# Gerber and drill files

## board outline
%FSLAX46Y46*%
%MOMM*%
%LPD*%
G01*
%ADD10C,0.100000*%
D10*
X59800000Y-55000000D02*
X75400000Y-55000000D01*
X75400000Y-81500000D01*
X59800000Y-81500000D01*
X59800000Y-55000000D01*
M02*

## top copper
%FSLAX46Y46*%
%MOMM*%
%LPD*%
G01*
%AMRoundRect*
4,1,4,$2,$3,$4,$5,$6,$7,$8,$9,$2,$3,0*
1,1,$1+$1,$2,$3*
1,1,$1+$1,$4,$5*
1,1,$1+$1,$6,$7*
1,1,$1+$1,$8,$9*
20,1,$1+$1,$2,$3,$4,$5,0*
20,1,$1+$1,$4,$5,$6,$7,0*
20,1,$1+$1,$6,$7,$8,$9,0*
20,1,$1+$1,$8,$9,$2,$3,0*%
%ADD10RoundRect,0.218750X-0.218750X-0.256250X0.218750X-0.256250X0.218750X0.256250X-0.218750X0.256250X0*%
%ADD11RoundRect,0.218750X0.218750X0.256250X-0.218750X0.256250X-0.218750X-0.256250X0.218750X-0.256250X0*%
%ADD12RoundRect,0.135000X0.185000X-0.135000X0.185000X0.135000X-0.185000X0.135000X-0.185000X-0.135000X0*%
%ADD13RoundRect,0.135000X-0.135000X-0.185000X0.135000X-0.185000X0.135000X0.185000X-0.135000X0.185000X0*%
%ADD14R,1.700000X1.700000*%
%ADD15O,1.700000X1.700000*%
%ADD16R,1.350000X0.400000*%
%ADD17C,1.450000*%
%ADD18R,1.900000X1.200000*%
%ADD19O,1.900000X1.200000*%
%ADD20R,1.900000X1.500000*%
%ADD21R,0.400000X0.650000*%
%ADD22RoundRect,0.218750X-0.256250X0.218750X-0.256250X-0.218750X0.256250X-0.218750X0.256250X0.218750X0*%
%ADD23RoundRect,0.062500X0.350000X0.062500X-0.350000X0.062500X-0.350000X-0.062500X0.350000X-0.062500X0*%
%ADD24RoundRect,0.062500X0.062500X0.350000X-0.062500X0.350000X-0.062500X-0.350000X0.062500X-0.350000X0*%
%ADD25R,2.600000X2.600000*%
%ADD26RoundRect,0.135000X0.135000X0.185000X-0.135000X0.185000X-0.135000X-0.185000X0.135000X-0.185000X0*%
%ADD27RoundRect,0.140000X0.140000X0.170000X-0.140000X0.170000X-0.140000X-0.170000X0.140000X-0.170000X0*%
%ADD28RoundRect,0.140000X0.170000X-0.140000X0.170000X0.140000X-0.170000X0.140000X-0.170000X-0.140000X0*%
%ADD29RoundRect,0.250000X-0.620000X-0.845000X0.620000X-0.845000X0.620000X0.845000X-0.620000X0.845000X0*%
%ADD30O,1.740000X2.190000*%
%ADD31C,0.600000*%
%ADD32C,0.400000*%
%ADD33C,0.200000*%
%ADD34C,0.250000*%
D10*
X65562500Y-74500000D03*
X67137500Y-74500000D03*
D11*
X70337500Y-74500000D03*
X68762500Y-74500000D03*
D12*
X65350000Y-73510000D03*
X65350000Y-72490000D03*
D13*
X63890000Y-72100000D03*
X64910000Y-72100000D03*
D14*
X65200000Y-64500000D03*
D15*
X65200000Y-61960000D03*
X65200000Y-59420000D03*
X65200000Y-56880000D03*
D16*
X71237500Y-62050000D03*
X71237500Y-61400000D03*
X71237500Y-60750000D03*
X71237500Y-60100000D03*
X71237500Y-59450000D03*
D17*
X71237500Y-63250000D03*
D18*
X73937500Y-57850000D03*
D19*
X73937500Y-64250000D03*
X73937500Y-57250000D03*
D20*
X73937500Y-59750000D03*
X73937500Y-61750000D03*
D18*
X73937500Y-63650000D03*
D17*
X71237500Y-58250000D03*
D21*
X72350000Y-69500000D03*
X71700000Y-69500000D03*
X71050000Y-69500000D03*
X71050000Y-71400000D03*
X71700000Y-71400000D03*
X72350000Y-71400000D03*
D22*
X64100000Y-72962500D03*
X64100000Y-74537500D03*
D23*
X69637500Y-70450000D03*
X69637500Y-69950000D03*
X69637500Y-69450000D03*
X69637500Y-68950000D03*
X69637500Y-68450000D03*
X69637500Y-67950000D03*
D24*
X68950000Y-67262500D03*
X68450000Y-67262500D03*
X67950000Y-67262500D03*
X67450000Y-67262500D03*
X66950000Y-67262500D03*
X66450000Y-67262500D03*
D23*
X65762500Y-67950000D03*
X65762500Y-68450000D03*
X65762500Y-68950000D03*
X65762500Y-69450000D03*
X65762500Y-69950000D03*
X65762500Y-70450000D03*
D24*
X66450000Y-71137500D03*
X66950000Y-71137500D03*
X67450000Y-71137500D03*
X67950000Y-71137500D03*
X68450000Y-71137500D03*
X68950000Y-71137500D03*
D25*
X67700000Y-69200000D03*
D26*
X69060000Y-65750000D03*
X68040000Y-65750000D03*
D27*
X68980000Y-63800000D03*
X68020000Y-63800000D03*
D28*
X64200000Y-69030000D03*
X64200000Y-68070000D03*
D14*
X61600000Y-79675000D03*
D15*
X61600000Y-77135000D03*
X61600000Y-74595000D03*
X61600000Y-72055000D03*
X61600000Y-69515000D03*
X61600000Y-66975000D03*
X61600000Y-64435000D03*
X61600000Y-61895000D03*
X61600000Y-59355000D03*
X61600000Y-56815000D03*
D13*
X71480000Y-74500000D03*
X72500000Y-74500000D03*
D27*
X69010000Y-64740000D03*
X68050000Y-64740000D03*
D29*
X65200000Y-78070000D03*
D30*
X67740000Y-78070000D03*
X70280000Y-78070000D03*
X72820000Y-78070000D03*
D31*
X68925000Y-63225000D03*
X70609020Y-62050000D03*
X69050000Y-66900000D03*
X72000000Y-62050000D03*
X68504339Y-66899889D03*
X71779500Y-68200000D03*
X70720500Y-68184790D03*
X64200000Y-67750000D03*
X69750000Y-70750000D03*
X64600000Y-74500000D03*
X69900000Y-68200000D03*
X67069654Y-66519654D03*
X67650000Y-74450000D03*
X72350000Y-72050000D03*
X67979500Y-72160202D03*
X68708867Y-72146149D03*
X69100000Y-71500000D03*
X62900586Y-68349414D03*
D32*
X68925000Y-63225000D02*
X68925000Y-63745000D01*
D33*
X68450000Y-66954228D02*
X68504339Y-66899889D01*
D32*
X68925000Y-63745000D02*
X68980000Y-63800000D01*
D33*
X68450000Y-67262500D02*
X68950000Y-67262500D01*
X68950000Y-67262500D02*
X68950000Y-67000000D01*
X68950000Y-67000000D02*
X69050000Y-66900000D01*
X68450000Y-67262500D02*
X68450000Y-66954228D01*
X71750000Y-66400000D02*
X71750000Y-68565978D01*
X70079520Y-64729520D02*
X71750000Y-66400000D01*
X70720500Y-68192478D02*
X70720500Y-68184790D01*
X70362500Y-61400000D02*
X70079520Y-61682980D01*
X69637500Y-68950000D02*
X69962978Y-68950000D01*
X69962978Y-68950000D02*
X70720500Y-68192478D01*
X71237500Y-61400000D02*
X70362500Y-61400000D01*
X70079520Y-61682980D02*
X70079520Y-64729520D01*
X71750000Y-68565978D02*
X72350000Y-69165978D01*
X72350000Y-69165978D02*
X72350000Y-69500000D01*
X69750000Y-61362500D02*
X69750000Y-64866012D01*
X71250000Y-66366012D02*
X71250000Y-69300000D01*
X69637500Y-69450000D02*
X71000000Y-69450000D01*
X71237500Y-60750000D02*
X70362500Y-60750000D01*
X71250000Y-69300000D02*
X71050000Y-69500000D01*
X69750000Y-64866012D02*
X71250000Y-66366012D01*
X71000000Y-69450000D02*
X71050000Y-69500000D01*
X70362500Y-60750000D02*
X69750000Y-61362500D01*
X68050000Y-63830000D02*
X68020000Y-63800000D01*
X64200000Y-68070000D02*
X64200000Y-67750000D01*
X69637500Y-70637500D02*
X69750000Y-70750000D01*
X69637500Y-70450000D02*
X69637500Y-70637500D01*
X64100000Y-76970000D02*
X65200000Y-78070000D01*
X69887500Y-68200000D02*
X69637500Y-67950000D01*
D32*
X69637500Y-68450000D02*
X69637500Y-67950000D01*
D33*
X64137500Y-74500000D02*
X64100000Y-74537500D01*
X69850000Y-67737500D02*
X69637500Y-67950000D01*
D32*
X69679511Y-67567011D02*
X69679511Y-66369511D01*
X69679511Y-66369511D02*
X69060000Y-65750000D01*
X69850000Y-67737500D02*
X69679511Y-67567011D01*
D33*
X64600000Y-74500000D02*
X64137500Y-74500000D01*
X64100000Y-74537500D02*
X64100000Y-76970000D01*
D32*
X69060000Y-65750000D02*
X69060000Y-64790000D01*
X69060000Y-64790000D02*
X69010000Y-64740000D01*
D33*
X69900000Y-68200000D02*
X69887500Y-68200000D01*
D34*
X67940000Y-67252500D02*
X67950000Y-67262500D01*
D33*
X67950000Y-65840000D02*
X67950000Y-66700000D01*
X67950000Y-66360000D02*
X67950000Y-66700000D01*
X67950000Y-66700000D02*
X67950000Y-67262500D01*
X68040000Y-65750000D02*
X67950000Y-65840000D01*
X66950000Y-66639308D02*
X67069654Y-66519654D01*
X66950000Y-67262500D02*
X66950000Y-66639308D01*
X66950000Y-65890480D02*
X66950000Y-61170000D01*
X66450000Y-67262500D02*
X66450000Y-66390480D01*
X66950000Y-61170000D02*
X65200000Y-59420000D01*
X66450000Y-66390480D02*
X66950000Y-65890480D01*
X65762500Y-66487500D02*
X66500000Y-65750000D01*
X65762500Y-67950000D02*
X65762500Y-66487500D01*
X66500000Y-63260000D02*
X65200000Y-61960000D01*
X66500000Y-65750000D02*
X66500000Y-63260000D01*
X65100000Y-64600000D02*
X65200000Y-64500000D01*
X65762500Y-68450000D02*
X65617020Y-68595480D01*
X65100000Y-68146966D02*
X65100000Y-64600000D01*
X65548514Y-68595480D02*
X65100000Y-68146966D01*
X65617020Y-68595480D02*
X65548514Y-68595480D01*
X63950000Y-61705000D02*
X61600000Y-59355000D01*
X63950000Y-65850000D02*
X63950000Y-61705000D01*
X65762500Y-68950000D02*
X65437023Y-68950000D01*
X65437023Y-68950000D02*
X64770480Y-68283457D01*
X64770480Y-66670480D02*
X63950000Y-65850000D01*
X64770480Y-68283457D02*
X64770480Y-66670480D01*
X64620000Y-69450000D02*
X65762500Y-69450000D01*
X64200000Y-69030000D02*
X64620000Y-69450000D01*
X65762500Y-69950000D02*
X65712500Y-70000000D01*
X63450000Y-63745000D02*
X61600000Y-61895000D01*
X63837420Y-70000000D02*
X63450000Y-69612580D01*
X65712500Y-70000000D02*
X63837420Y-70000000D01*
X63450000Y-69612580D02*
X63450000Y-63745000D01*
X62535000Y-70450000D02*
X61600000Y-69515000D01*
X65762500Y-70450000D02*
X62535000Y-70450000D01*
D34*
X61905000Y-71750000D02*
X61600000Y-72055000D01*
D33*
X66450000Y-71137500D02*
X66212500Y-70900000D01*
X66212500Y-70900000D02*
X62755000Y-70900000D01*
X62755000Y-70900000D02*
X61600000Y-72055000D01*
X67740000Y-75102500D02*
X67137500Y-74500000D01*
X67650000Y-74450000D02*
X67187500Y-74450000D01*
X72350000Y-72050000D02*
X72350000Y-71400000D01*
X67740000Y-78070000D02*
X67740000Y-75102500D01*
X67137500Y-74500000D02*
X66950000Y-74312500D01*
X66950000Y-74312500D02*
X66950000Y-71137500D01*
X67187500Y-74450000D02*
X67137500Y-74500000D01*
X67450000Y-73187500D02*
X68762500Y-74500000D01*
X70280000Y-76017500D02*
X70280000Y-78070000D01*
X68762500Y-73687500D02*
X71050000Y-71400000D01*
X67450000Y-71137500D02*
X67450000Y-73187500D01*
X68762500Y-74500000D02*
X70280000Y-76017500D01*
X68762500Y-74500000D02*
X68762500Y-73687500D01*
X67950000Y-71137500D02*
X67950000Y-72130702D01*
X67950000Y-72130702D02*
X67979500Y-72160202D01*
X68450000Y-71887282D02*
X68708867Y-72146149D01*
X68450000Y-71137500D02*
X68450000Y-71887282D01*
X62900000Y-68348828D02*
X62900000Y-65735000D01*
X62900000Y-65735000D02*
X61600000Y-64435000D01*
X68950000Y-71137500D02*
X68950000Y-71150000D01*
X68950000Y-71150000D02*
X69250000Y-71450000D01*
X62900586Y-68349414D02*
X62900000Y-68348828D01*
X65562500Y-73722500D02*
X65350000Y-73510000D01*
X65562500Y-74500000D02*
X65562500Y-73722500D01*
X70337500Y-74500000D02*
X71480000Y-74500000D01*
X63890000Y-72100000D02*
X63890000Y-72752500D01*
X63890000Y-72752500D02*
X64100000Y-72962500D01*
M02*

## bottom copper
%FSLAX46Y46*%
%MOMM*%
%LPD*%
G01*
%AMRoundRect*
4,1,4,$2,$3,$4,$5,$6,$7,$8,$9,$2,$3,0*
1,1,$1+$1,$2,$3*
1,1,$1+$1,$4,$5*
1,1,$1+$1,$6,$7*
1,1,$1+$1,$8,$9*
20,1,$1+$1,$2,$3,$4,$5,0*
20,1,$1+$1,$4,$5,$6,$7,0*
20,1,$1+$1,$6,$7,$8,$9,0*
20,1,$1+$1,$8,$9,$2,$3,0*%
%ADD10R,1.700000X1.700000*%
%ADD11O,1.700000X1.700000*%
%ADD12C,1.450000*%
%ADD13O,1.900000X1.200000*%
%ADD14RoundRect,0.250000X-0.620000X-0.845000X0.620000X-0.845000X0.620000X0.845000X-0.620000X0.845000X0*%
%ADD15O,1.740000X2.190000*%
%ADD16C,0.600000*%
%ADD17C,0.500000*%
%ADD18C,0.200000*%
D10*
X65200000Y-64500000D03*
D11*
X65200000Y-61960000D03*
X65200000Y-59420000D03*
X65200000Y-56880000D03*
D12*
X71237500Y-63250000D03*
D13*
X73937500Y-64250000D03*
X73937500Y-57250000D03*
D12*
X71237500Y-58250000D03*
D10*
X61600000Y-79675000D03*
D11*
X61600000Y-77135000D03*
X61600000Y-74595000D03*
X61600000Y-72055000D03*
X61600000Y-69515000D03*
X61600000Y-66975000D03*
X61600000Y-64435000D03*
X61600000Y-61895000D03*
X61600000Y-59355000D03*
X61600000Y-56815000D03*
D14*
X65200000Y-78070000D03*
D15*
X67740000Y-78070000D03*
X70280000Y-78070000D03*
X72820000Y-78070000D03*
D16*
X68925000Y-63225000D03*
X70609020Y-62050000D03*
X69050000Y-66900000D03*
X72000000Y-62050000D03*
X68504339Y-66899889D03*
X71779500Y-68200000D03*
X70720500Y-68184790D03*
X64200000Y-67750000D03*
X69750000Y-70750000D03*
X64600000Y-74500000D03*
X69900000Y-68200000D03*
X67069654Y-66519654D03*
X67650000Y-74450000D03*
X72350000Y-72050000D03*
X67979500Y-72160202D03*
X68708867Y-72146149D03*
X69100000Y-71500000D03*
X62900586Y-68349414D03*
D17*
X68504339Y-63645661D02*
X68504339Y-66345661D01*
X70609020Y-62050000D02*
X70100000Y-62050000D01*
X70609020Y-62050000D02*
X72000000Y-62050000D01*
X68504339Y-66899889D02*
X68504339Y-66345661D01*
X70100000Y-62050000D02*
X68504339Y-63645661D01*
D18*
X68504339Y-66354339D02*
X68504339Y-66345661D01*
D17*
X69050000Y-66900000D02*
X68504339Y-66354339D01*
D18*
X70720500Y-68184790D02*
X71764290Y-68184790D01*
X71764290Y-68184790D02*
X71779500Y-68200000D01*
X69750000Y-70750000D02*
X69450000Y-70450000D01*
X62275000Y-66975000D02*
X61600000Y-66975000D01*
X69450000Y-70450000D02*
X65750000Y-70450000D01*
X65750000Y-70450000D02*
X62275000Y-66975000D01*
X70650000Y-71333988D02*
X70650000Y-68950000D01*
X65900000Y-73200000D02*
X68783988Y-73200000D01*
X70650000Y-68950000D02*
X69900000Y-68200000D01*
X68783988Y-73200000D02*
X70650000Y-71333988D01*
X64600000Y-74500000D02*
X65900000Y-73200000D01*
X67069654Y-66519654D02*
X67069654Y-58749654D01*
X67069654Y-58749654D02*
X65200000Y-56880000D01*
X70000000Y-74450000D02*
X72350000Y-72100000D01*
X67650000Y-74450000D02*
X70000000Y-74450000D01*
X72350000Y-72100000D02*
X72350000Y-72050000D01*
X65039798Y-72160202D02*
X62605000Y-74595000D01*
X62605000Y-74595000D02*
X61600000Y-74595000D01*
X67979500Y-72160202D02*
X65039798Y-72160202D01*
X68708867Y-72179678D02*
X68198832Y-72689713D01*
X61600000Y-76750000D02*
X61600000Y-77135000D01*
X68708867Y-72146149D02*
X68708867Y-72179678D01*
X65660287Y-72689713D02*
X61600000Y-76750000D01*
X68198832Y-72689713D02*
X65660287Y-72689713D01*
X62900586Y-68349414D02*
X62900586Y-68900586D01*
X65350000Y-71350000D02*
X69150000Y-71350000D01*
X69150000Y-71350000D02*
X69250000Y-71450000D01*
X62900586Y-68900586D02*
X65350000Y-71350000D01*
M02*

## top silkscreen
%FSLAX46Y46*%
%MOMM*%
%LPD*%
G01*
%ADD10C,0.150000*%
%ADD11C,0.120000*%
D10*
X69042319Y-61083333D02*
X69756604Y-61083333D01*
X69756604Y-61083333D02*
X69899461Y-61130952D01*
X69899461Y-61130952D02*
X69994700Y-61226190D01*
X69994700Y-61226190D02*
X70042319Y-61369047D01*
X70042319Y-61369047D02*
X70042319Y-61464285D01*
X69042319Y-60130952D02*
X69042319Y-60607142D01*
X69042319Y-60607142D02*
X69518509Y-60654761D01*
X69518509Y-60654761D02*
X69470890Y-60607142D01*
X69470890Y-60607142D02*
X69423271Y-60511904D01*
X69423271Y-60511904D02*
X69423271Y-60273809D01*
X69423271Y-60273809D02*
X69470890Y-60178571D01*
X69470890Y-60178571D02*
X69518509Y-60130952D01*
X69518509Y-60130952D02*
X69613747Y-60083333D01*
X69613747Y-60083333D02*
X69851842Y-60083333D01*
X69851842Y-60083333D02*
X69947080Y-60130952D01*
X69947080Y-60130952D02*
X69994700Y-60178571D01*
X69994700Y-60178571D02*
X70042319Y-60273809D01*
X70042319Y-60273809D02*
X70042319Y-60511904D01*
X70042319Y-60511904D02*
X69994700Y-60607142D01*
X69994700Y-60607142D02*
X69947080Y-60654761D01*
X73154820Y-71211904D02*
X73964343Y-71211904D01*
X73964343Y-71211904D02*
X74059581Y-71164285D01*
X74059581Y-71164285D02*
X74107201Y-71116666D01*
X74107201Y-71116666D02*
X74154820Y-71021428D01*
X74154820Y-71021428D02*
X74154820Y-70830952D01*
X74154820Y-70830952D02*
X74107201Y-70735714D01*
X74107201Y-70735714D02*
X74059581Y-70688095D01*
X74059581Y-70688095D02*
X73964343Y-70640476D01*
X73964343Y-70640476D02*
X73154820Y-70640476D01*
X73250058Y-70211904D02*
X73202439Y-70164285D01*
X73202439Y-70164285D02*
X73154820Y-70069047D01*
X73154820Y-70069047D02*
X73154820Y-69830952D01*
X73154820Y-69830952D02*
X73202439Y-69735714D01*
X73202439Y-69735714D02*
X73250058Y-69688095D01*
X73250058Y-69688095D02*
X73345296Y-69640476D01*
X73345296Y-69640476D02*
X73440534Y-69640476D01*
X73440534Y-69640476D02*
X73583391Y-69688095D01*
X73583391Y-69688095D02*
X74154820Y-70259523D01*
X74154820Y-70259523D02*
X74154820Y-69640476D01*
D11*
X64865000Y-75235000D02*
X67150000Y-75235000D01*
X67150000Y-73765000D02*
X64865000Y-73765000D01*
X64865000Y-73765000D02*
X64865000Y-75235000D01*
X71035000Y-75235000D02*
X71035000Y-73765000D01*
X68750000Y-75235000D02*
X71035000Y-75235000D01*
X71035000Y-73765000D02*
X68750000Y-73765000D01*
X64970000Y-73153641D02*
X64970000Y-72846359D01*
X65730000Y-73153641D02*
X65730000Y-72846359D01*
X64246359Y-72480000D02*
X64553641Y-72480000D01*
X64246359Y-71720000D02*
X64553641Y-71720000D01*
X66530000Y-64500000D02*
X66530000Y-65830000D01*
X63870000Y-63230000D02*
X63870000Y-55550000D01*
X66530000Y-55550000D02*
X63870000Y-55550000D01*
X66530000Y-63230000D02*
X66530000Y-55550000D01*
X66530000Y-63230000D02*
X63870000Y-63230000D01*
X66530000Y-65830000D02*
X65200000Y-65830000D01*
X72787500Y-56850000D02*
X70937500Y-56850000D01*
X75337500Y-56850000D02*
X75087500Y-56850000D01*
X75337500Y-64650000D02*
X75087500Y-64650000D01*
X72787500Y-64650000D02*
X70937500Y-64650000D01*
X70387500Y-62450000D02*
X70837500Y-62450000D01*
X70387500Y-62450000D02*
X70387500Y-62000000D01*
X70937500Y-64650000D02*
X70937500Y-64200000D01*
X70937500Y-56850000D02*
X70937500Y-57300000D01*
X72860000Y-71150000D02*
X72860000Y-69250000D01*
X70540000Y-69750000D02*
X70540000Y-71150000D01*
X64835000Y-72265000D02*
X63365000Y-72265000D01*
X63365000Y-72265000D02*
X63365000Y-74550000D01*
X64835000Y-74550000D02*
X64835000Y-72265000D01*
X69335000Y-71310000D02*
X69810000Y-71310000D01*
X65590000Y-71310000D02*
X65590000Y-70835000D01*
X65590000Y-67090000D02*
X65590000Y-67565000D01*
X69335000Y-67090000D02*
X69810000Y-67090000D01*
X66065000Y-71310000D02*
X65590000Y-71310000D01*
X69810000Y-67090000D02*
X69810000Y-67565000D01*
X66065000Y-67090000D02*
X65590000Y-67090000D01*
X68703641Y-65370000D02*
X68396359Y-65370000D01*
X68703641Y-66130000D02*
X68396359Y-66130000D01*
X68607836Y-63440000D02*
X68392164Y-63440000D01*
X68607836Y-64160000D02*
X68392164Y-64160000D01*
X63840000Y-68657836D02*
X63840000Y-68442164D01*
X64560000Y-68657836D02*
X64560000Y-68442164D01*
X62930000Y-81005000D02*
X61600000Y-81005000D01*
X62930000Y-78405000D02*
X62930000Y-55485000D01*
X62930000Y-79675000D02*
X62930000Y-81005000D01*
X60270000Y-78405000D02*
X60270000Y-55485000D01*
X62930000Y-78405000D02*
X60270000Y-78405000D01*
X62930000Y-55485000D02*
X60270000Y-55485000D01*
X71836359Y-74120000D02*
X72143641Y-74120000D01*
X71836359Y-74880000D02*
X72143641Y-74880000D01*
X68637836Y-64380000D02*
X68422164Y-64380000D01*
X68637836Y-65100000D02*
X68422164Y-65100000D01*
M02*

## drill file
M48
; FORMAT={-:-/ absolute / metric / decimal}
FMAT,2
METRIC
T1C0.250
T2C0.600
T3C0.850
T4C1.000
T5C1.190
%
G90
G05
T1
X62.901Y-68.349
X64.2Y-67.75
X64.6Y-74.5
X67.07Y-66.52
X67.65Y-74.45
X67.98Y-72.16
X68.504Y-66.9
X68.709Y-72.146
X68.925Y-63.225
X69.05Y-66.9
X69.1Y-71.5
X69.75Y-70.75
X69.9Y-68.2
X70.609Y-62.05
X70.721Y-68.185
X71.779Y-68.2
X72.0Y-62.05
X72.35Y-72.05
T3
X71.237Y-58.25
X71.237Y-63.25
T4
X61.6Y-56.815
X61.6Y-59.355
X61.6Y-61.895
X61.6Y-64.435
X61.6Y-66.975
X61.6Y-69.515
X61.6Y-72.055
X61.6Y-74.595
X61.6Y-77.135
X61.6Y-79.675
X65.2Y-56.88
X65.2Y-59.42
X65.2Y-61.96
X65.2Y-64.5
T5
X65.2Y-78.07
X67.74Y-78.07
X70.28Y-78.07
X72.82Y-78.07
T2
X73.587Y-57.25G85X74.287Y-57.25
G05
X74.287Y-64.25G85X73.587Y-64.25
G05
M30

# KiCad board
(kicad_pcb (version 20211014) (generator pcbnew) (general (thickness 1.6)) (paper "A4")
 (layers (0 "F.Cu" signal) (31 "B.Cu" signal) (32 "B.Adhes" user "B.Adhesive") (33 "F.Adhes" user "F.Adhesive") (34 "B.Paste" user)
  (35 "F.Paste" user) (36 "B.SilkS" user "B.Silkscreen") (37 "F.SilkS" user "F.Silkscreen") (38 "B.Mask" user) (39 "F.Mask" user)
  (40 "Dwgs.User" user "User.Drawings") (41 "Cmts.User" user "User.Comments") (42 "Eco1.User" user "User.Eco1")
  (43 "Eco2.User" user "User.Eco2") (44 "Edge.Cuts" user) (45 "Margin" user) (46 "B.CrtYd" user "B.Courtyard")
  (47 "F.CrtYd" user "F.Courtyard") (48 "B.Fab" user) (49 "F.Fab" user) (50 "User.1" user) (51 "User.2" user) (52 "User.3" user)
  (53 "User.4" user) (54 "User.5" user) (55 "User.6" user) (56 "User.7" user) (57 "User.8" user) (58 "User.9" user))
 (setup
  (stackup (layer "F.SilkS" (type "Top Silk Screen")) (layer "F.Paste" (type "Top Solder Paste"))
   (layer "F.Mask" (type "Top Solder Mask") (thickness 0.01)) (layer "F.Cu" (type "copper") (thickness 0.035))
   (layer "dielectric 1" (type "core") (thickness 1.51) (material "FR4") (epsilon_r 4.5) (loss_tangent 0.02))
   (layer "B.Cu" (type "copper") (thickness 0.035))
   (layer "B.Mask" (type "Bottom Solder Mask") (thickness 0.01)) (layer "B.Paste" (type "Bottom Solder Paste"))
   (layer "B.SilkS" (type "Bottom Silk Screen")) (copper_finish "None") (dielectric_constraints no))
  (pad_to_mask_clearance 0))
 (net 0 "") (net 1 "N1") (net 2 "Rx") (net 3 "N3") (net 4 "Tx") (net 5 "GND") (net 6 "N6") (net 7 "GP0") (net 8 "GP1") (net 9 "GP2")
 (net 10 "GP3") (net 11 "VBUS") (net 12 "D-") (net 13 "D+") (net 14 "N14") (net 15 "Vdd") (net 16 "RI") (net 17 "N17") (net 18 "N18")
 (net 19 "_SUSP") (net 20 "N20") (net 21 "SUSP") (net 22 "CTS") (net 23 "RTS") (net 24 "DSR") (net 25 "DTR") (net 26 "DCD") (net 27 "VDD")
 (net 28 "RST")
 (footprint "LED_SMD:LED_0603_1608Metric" (layer "F.Cu") (at 66.35 74.5)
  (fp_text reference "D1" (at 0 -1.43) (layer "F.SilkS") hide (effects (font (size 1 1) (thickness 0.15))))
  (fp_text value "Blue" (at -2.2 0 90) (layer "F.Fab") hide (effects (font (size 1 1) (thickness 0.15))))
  (fp_line (start -1.485 0.735) (end 0.8 0.735) (layer "F.SilkS") (width 0.12))
  (fp_line (start 0.8 -0.735) (end -1.485 -0.735) (layer "F.SilkS") (width 0.12))
  (fp_line (start -1.485 -0.735) (end -1.485 0.735) (layer "F.SilkS") (width 0.12))
  (pad "1" smd roundrect locked (at -0.7875 0) (size 0.875 0.95) (layers "F.Cu" "F.Paste" "F.Mask") (roundrect_rratio 0.25) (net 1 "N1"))
  (pad "2" smd roundrect locked (at 0.7875 0) (size 0.875 0.95) (layers "F.Cu" "F.Paste" "F.Mask") (roundrect_rratio 0.25) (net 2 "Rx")))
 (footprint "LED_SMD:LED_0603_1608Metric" (layer "F.Cu") (at 69.55 74.5 180)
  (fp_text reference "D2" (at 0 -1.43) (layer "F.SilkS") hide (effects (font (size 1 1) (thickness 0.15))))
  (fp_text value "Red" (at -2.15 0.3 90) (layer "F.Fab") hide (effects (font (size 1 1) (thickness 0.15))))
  (fp_line (start -1.485 -0.735) (end -1.485 0.735) (layer "F.SilkS") (width 0.12))
  (fp_line (start 0.8 -0.735) (end -1.485 -0.735) (layer "F.SilkS") (width 0.12))
  (fp_line (start -1.485 0.735) (end 0.8 0.735) (layer "F.SilkS") (width 0.12))
  (pad "1" smd roundrect locked (at -0.7875 0 180) (size 0.875 0.95) (layers "F.Cu" "F.Paste" "F.Mask") (roundrect_rratio 0.25) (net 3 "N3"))
  (pad "2" smd roundrect locked (at 0.7875 0 180) (size 0.875 0.95) (layers "F.Cu" "F.Paste" "F.Mask") (roundrect_rratio 0.25) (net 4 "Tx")))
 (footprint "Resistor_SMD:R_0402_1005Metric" (layer "F.Cu") (at 65.35 73 90)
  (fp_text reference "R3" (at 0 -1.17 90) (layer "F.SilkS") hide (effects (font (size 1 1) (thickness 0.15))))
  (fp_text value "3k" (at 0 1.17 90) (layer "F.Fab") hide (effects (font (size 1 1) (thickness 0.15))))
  (fp_line (start -0.153641 -0.38) (end 0.153641 -0.38) (layer "F.SilkS") (width 0.12))
  (fp_line (start -0.153641 0.38) (end 0.153641 0.38) (layer "F.SilkS") (width 0.12))
  (pad "1" smd roundrect locked (at -0.51 0 90) (size 0.54 0.64) (layers "F.Cu" "F.Paste" "F.Mask") (roundrect_rratio 0.25) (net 1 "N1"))
  (pad "2" smd roundrect locked (at 0.51 0 90) (size 0.54 0.64) (layers "F.Cu" "F.Paste" "F.Mask") (roundrect_rratio 0.25) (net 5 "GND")))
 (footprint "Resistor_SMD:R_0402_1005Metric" (layer "F.Cu") (at 64.4 72.1)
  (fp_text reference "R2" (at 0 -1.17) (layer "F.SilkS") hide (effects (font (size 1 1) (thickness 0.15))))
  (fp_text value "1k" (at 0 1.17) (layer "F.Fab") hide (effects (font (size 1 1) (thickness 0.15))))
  (fp_line (start -0.153641 0.38) (end 0.153641 0.38) (layer "F.SilkS") (width 0.12))
  (fp_line (start -0.153641 -0.38) (end 0.153641 -0.38) (layer "F.SilkS") (width 0.12))
  (pad "1" smd roundrect locked (at -0.51 0) (size 0.54 0.64) (layers "F.Cu" "F.Paste" "F.Mask") (roundrect_rratio 0.25) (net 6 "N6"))
  (pad "2" smd roundrect locked (at 0.51 0) (size 0.54 0.64) (layers "F.Cu" "F.Paste" "F.Mask") (roundrect_rratio 0.25) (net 5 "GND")))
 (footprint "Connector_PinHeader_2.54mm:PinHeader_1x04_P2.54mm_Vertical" (layer "F.Cu") (at 65.2 64.5 180)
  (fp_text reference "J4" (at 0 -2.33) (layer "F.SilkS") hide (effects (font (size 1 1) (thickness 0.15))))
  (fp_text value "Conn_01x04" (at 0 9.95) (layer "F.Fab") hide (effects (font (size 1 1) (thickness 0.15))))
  (fp_line (start -1.33 0) (end -1.33 -1.33) (layer "F.SilkS") (width 0.12))
  (fp_line (start 1.33 1.27) (end 1.33 8.95) (layer "F.SilkS") (width 0.12))
  (fp_line (start -1.33 8.95) (end 1.33 8.95) (layer "F.SilkS") (width 0.12))
  (fp_line (start -1.33 1.27) (end -1.33 8.95) (layer "F.SilkS") (width 0.12))
  (fp_line (start -1.33 1.27) (end 1.33 1.27) (layer "F.SilkS") (width 0.12))
  (fp_line (start -1.33 -1.33) (end 0 -1.33) (layer "F.SilkS") (width 0.12))
  (pad "1" thru_hole rect locked (at 0 0 180) (size 1.7 1.7) (drill 1) (layers *.Cu *.Mask) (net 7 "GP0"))
  (pad "2" thru_hole oval locked (at 0 2.54 180) (size 1.7 1.7) (drill 1) (layers *.Cu *.Mask) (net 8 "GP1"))
  (pad "3" thru_hole oval locked (at 0 5.08 180) (size 1.7 1.7) (drill 1) (layers *.Cu *.Mask) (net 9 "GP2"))
  (pad "4" thru_hole oval locked (at 0 7.62 180) (size 1.7 1.7) (drill 1) (layers *.Cu *.Mask) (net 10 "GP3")))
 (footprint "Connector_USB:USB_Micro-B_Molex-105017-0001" (layer "F.Cu") (at 72.7 60.75 90)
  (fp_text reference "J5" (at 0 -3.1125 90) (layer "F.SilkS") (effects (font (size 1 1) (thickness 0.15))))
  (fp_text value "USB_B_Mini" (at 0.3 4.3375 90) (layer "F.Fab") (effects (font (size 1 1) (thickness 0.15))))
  (fp_line (start 3.9 0.0875) (end 3.9 -1.7625) (layer "F.SilkS") (width 0.12))
  (fp_line (start 3.9 2.6375) (end 3.9 2.3875) (layer "F.SilkS") (width 0.12))
  (fp_line (start -3.9 2.6375) (end -3.9 2.3875) (layer "F.SilkS") (width 0.12))
  (fp_line (start -3.9 0.0875) (end -3.9 -1.7625) (layer "F.SilkS") (width 0.12))
  (fp_line (start -1.7 -2.3125) (end -1.7 -1.8625) (layer "F.SilkS") (width 0.12))
  (fp_line (start -1.7 -2.3125) (end -1.25 -2.3125) (layer "F.SilkS") (width 0.12))
  (fp_line (start -3.9 -1.7625) (end -3.45 -1.7625) (layer "F.SilkS") (width 0.12))
  (fp_line (start 3.9 -1.7625) (end 3.45 -1.7625) (layer "F.SilkS") (width 0.12))
  (pad "1" smd rect locked (at -1.3 -1.4625 90) (size 0.4 1.35) (layers "F.Cu" "F.Paste" "F.Mask") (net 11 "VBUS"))
  (pad "2" smd rect locked (at -0.65 -1.4625 90) (size 0.4 1.35) (layers "F.Cu" "F.Paste" "F.Mask") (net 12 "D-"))
  (pad "3" smd rect locked (at 0 -1.4625 90) (size 0.4 1.35) (layers "F.Cu" "F.Paste" "F.Mask") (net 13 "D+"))
  (pad "4" smd rect locked (at 0.65 -1.4625 90) (size 0.4 1.35) (layers "F.Cu" "F.Paste" "F.Mask") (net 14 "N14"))
  (pad "5" smd rect locked (at 1.3 -1.4625 90) (size 0.4 1.35) (layers "F.Cu" "F.Paste" "F.Mask") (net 5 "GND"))
  (pad "6" thru_hole circle locked (at -2.5 -1.4625 90) (size 1.45 1.45) (drill 0.85) (layers *.Cu *.Mask) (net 5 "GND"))
  (pad "6" smd rect locked (at 2.9 1.2375 90) (size 1.2 1.9) (layers "F.Cu" "F.Mask") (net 5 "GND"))
  (pad "6" thru_hole oval locked (at -3.5 1.2375 270) (size 1.2 1.9) (drill oval 0.6 1.3) (layers *.Cu *.Mask) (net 5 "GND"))
  (pad "6" thru_hole oval locked (at 3.5 1.2375 90) (size 1.2 1.9) (drill oval 0.6 1.3) (layers *.Cu *.Mask) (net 5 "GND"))
  (pad "6" smd rect locked (at 1 1.2375 90) (size 1.5 1.9) (layers "F.Cu" "F.Paste" "F.Mask") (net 5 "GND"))
  (pad "6" smd rect locked (at -1 1.2375 90) (size 1.5 1.9) (layers "F.Cu" "F.Paste" "F.Mask") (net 5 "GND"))
  (pad "6" smd rect locked (at -2.9 1.2375 90) (size 1.2 1.9) (layers "F.Cu" "F.Mask") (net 5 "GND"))
  (pad "6" thru_hole circle locked (at 2.5 -1.4625 90) (size 1.45 1.45) (drill 0.85) (layers *.Cu *.Mask) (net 5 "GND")))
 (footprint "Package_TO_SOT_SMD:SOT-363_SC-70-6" (layer "F.Cu") (at 71.7 70.45 -90)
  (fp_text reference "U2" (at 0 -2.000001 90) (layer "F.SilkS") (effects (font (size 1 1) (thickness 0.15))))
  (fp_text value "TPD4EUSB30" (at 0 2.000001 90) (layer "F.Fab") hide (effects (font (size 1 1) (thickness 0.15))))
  (fp_line (start 0.7 -1.16) (end -1.2 -1.16) (layer "F.SilkS") (width 0.12))
  (fp_line (start -0.7 1.16) (end 0.7 1.16) (layer "F.SilkS") (width 0.12))
  (pad "1" smd rect locked (at -0.95 -0.65 270) (size 0.65 0.4) (layers "F.Cu" "F.Paste" "F.Mask") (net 12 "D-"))
  (pad "2" smd rect locked (at -0.95 0 270) (size 0.65 0.4) (layers "F.Cu" "F.Paste" "F.Mask") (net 5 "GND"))
  (pad "3" smd rect locked (at -0.95 0.65 270) (size 0.65 0.4) (layers "F.Cu" "F.Paste" "F.Mask") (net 13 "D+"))
  (pad "4" smd rect locked (at 0.95 0.65 270) (size 0.65 0.4) (layers "F.Cu" "F.Paste" "F.Mask") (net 4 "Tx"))
  (pad "5" smd rect locked (at 0.95 0 270) (size 0.65 0.4) (layers "F.Cu" "F.Paste" "F.Mask"))
  (pad "6" smd rect locked (at 0.95 -0.65 270) (size 0.65 0.4) (layers "F.Cu" "F.Paste" "F.Mask") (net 2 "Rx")))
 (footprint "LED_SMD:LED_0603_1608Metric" (layer "F.Cu") (at 64.1 73.75 -90)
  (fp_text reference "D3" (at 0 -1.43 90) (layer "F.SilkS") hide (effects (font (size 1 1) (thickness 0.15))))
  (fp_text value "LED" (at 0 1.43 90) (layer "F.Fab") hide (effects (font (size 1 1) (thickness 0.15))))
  (fp_line (start -1.485 -0.735) (end -1.485 0.735) (layer "F.SilkS") (width 0.12))
  (fp_line (start -1.485 0.735) (end 0.8 0.735) (layer "F.SilkS") (width 0.12))
  (fp_line (start 0.8 -0.735) (end -1.485 -0.735) (layer "F.SilkS") (width 0.12))
  (pad "1" smd roundrect locked (at -0.7875 0 270) (size 0.875 0.95) (layers "F.Cu" "F.Paste" "F.Mask") (roundrect_rratio 0.25) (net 6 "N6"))
  (pad "2" smd roundrect locked (at 0.7875 0 270) (size 0.875 0.95) (layers "F.Cu" "F.Paste" "F.Mask") (roundrect_rratio 0.25)
   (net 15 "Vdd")))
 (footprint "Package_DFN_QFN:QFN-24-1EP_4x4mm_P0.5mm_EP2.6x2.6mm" (layer "F.Cu") (at 67.7 69.2 180)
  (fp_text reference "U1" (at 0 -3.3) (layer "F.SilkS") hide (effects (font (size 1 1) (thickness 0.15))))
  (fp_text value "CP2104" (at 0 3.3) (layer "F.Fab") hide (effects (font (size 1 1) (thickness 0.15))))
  (fp_line (start -1.635 -2.11) (end -2.11 -2.11) (layer "F.SilkS") (width 0.12))
  (fp_line (start 2.11 -2.11) (end 2.11 -1.635) (layer "F.SilkS") (width 0.12))
  (fp_line (start 2.11 2.11) (end 2.11 1.635) (layer "F.SilkS") (width 0.12))
  (fp_line (start -1.635 2.11) (end -2.11 2.11) (layer "F.SilkS") (width 0.12))
  (fp_line (start 1.635 -2.11) (end 2.11 -2.11) (layer "F.SilkS") (width 0.12))
  (fp_line (start -2.11 2.11) (end -2.11 1.635) (layer "F.SilkS") (width 0.12))
  (fp_line (start 1.635 2.11) (end 2.11 2.11) (layer "F.SilkS") (width 0.12))
  (pad "" smd roundrect locked (at -0.65 -0.65 180) (size 1.05 1.05) (layers "F.Paste") (roundrect_rratio 0.238095))
  (pad "" smd roundrect locked (at 0.65 -0.65 180) (size 1.05 1.05) (layers "F.Paste") (roundrect_rratio 0.238095))
  (pad "" smd roundrect locked (at 0.65 0.65 180) (size 1.05 1.05) (layers "F.Paste") (roundrect_rratio 0.238095))
  (pad "" smd roundrect locked (at -0.65 0.65 180) (size 1.05 1.05) (layers "F.Paste") (roundrect_rratio 0.238095))
  (pad "1" smd roundrect locked (at -1.9375 -1.25 180) (size 0.825 0.25) (layers "F.Cu" "F.Paste" "F.Mask") (roundrect_rratio 0.25)
   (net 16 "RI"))
  (pad "2" smd roundrect locked (at -1.9375 -0.75 180) (size 0.825 0.25) (layers "F.Cu" "F.Paste" "F.Mask") (roundrect_rratio 0.25)
   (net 5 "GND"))
  (pad "3" smd roundrect locked (at -1.9375 -0.25 180) (size 0.825 0.25) (layers "F.Cu" "F.Paste" "F.Mask") (roundrect_rratio 0.25)
   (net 13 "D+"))
  (pad "4" smd roundrect locked (at -1.9375 0.25 180) (size 0.825 0.25) (layers "F.Cu" "F.Paste" "F.Mask") (roundrect_rratio 0.25)
   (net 12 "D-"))
  (pad "5" smd roundrect locked (at -1.9375 0.75 180) (size 0.825 0.25) (layers "F.Cu" "F.Paste" "F.Mask") (roundrect_rratio 0.25)
   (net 15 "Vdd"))
  (pad "6" smd roundrect locked (at -1.9375 1.25 180) (size 0.825 0.25) (layers "F.Cu" "F.Paste" "F.Mask") (roundrect_rratio 0.25)
   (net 15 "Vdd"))
  (pad "7" smd roundrect locked (at -1.25 1.9375 180) (size 0.25 0.825) (layers "F.Cu" "F.Paste" "F.Mask") (roundrect_rratio 0.25)
   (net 11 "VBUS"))
  (pad "8" smd roundrect locked (at -0.75 1.9375 180) (size 0.25 0.825) (layers "F.Cu" "F.Paste" "F.Mask") (roundrect_rratio 0.25)
   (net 11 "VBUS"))
  (pad "9" smd roundrect locked (at -0.25 1.9375 180) (size 0.25 0.825) (layers "F.Cu" "F.Paste" "F.Mask") (roundrect_rratio 0.25)
   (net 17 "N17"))
  (pad "10" smd roundrect locked (at 0.25 1.9375 180) (size 0.25 0.825) (layers "F.Cu" "F.Paste" "F.Mask") (roundrect_rratio 0.25)
   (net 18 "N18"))
  (pad "11" smd roundrect locked (at 0.75 1.9375 180) (size 0.25 0.825) (layers "F.Cu" "F.Paste" "F.Mask") (roundrect_rratio 0.25)
   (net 10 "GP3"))
  (pad "12" smd roundrect locked (at 1.25 1.9375 180) (size 0.25 0.825) (layers "F.Cu" "F.Paste" "F.Mask") (roundrect_rratio 0.25)
   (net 9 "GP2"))
  (pad "13" smd roundrect locked (at 1.9375 1.25 180) (size 0.825 0.25) (layers "F.Cu" "F.Paste" "F.Mask") (roundrect_rratio 0.25)
   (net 8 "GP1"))
  (pad "14" smd roundrect locked (at 1.9375 0.75 180) (size 0.825 0.25) (layers "F.Cu" "F.Paste" "F.Mask") (roundrect_rratio 0.25)
   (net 7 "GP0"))
  (pad "15" smd roundrect locked (at 1.9375 0.25 180) (size 0.825 0.25) (layers "F.Cu" "F.Paste" "F.Mask") (roundrect_rratio 0.25)
   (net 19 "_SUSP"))
  (pad "16" smd roundrect locked (at 1.9375 -0.25 180) (size 0.825 0.25) (layers "F.Cu" "F.Paste" "F.Mask") (roundrect_rratio 0.25)
   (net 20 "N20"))
  (pad "17" smd roundrect locked (at 1.9375 -0.75 180) (size 0.825 0.25) (layers "F.Cu" "F.Paste" "F.Mask") (roundrect_rratio 0.25)
   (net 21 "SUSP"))
  (pad "18" smd roundrect locked (at 1.9375 -1.25 180) (size 0.825 0.25) (layers "F.Cu" "F.Paste" "F.Mask") (roundrect_rratio 0.25)
   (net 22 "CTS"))
  (pad "19" smd roundrect locked (at 1.25 -1.9375 180) (size 0.25 0.825) (layers "F.Cu" "F.Paste" "F.Mask") (roundrect_rratio 0.25)
   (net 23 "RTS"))
  (pad "20" smd roundrect locked (at 0.75 -1.9375 180) (size 0.25 0.825) (layers "F.Cu" "F.Paste" "F.Mask") (roundrect_rratio 0.25)
   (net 2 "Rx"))
  (pad "21" smd roundrect locked (at 0.25 -1.9375 180) (size 0.25 0.825) (layers "F.Cu" "F.Paste" "F.Mask") (roundrect_rratio 0.25)
   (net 4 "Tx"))
  (pad "22" smd roundrect locked (at -0.25 -1.9375 180) (size 0.25 0.825) (layers "F.Cu" "F.Paste" "F.Mask") (roundrect_rratio 0.25)
   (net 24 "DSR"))
  (pad "23" smd roundrect locked (at -0.75 -1.9375 180) (size 0.25 0.825) (layers "F.Cu" "F.Paste" "F.Mask") (roundrect_rratio 0.25)
   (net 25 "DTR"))
  (pad "24" smd roundrect locked (at -1.25 -1.9375 180) (size 0.25 0.825) (layers "F.Cu" "F.Paste" "F.Mask") (roundrect_rratio 0.25)
   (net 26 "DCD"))
  (pad "25" smd rect locked (at 0 0 180) (size 2.6 2.6) (layers "F.Cu" "F.Mask") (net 5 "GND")))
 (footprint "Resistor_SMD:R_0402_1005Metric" (layer "F.Cu") (at 68.55 65.75 180)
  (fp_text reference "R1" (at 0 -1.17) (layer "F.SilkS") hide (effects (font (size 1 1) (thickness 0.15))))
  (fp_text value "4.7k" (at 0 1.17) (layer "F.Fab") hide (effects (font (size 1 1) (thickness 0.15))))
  (fp_line (start -0.153641 0.38) (end 0.153641 0.38) (layer "F.SilkS") (width 0.12))
  (fp_line (start -0.153641 -0.38) (end 0.153641 -0.38) (layer "F.SilkS") (width 0.12))
  (pad "1" smd roundrect locked (at -0.51 0 180) (size 0.54 0.64) (layers "F.Cu" "F.Paste" "F.Mask") (roundrect_rratio 0.25) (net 15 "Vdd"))
  (pad "2" smd roundrect locked (at 0.51 0 180) (size 0.54 0.64) (layers "F.Cu" "F.Paste" "F.Mask") (roundrect_rratio 0.25) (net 17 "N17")))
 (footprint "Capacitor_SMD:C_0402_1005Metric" (layer "F.Cu") (at 68.5 63.8 180)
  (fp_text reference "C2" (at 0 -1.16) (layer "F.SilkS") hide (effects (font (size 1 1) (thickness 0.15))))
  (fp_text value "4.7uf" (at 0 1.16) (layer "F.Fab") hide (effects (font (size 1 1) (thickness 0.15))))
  (fp_line (start -0.107836 0.36) (end 0.107836 0.36) (layer "F.SilkS") (width 0.12))
  (fp_line (start -0.107836 -0.36) (end 0.107836 -0.36) (layer "F.SilkS") (width 0.12))
  (pad "1" smd roundrect locked (at -0.48 0 180) (size 0.56 0.62) (layers "F.Cu" "F.Paste" "F.Mask") (roundrect_rratio 0.25) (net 11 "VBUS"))
  (pad "2" smd roundrect locked (at 0.48 0 180) (size 0.56 0.62) (layers "F.Cu" "F.Paste" "F.Mask") (roundrect_rratio 0.25) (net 5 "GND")))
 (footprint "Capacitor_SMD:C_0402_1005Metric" (layer "F.Cu") (at 64.2 68.55 90)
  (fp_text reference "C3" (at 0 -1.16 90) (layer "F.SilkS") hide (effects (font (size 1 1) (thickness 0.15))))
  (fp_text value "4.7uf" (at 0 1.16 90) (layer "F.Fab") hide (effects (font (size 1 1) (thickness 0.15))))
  (fp_line (start -0.107836 -0.36) (end 0.107836 -0.36) (layer "F.SilkS") (width 0.12))
  (fp_line (start -0.107836 0.36) (end 0.107836 0.36) (layer "F.SilkS") (width 0.12))
  (pad "1" smd roundrect locked (at -0.48 0 90) (size 0.56 0.62) (layers "F.Cu" "F.Paste" "F.Mask") (roundrect_rratio 0.25) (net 20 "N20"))
  (pad "2" smd roundrect locked (at 0.48 0 90) (size 0.56 0.62) (layers "F.Cu" "F.Paste" "F.Mask") (roundrect_rratio 0.25) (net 5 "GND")))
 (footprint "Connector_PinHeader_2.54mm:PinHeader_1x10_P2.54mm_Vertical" (layer "F.Cu") (at 61.6 79.675 180)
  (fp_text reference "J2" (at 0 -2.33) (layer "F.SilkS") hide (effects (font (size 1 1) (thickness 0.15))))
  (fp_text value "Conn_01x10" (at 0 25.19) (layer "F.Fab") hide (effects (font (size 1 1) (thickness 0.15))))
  (fp_line (start -1.33 -1.33) (end 0 -1.33) (layer "F.SilkS") (width 0.12))
  (fp_line (start -1.33 1.27) (end -1.33 24.19) (layer "F.SilkS") (width 0.12))
  (fp_line (start -1.33 0) (end -1.33 -1.33) (layer "F.SilkS") (width 0.12))
  (fp_line (start 1.33 1.27) (end 1.33 24.19) (layer "F.SilkS") (width 0.12))
  (fp_line (start -1.33 1.27) (end 1.33 1.27) (layer "F.SilkS") (width 0.12))
  (fp_line (start -1.33 24.19) (end 1.33 24.19) (layer "F.SilkS") (width 0.12))
  (pad "1" thru_hole rect locked (at 0 0 180) (size 1.7 1.7) (drill 1) (layers *.Cu *.Mask) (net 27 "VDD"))
  (pad "2" thru_hole oval locked (at 0 2.54 180) (size 1.7 1.7) (drill 1) (layers *.Cu *.Mask) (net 25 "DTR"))
  (pad "3" thru_hole oval locked (at 0 5.08 180) (size 1.7 1.7) (drill 1) (layers *.Cu *.Mask) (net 24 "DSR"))
  (pad "4" thru_hole oval locked (at 0 7.62 180) (size 1.7 1.7) (drill 1) (layers *.Cu *.Mask) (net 23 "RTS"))
  (pad "5" thru_hole oval locked (at 0 10.16 180) (size 1.7 1.7) (drill 1) (layers *.Cu *.Mask) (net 22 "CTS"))
  (pad "6" thru_hole oval locked (at 0 12.7 180) (size 1.7 1.7) (drill 1) (layers *.Cu *.Mask) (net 16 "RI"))
  (pad "7" thru_hole oval locked (at 0 15.24 180) (size 1.7 1.7) (drill 1) (layers *.Cu *.Mask) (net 26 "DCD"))
  (pad "8" thru_hole oval locked (at 0 17.78 180) (size 1.7 1.7) (drill 1) (layers *.Cu *.Mask) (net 21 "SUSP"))
  (pad "9" thru_hole oval locked (at 0 20.32 180) (size 1.7 1.7) (drill 1) (layers *.Cu *.Mask) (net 19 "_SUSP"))
  (pad "10" thru_hole oval locked (at 0 22.86 180) (size 1.7 1.7) (drill 1) (layers *.Cu *.Mask) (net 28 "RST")))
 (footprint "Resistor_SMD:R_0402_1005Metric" (layer "F.Cu") (at 71.99 74.5)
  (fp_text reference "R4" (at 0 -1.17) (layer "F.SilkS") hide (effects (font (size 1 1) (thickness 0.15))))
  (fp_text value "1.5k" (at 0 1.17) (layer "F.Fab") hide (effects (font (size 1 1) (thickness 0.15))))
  (fp_line (start -0.153641 -0.38) (end 0.153641 -0.38) (layer "F.SilkS") (width 0.12))
  (fp_line (start -0.153641 0.38) (end 0.153641 0.38) (layer "F.SilkS") (width 0.12))
  (pad "1" smd roundrect locked (at -0.51 0) (size 0.54 0.64) (layers "F.Cu" "F.Paste" "F.Mask") (roundrect_rratio 0.25) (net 3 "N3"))
  (pad "2" smd roundrect locked (at 0.51 0) (size 0.54 0.64) (layers "F.Cu" "F.Paste" "F.Mask") (roundrect_rratio 0.25) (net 5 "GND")))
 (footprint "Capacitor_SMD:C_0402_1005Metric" (layer "F.Cu") (at 68.53 64.74 180)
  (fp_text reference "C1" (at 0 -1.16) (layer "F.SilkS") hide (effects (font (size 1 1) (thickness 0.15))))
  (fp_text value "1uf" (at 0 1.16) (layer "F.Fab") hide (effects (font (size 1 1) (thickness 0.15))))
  (fp_line (start -0.107836 0.36) (end 0.107836 0.36) (layer "F.SilkS") (width 0.12))
  (fp_line (start -0.107836 -0.36) (end 0.107836 -0.36) (layer "F.SilkS") (width 0.12))
  (pad "1" smd roundrect locked (at -0.48 0 180) (size 0.56 0.62) (layers "F.Cu" "F.Paste" "F.Mask") (roundrect_rratio 0.25) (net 15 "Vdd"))
  (pad "2" smd roundrect locked (at 0.48 0 180) (size 0.56 0.62) (layers "F.Cu" "F.Paste" "F.Mask") (roundrect_rratio 0.25) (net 5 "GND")))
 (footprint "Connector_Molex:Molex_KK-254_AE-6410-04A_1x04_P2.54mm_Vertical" (layer "B.Cu") (at 65.2 78.07)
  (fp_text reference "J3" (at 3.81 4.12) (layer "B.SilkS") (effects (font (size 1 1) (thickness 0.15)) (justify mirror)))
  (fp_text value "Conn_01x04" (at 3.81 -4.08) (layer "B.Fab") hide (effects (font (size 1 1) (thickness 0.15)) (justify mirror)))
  (pad "1" thru_hole roundrect locked (at 0 0) (size 1.74 2.19) (drill 1.19) (layers *.Cu *.Mask) (roundrect_rratio 0.143678) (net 15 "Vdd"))
  (pad "2" thru_hole oval locked (at 2.54 0) (size 1.74 2.19) (drill 1.19) (layers *.Cu *.Mask) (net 2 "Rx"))
  (pad "3" thru_hole oval locked (at 5.08 0) (size 1.74 2.19) (drill 1.19) (layers *.Cu *.Mask) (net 4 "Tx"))
  (pad "4" thru_hole oval locked (at 7.62 0) (size 1.74 2.19) (drill 1.19) (layers *.Cu *.Mask) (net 5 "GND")))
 (gr_rect (start 59.8 55) (end 75.4 81.5) (layer "Edge.Cuts") (width 0.1) (fill none))
 (segment (start 68.925 63.225) (end 68.925 63.745) (width 0.4) (layer "F.Cu") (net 11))
 (segment (start 68.45 66.954228) (end 68.504339 66.899889) (width 0.2) (layer "F.Cu") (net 11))
 (segment (start 68.925 63.745) (end 68.98 63.8) (width 0.4) (layer "F.Cu") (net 11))
 (segment (start 68.45 67.2625) (end 68.95 67.2625) (width 0.2) (layer "F.Cu") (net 11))
 (segment (start 68.95 67.2625) (end 68.95 67) (width 0.2) (layer "F.Cu") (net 11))
 (segment (start 68.95 67) (end 69.05 66.9) (width 0.2) (layer "F.Cu") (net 11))
 (segment (start 68.45 67.2625) (end 68.45 66.954228) (width 0.2) (layer "F.Cu") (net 11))
 (via (at 68.925 63.225) (size 0.6) (drill 0.25) (layers "F.Cu" "B.Cu") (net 11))
 (via (at 70.60902 62.05) (size 0.6) (drill 0.25) (layers "F.Cu" "B.Cu") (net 11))
 (via (at 69.05 66.9) (size 0.6) (drill 0.25) (layers "F.Cu" "B.Cu") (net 11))
 (via (at 72 62.05) (size 0.6) (drill 0.25) (layers "F.Cu" "B.Cu") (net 11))
 (via (at 68.504339 66.899889) (size 0.6) (drill 0.25) (layers "F.Cu" "B.Cu") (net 11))
 (segment (start 68.504339 63.645661) (end 68.504339 66.345661) (width 0.5) (layer "B.Cu") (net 11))
 (segment (start 70.60902 62.05) (end 70.1 62.05) (width 0.5) (layer "B.Cu") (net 11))
 (segment (start 70.60902 62.05) (end 72 62.05) (width 0.5) (layer "B.Cu") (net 11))
 (segment (start 68.504339 66.899889) (end 68.504339 66.345661) (width 0.5) (layer "B.Cu") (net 11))
 (segment (start 70.1 62.05) (end 68.504339 63.645661) (width 0.5) (layer "B.Cu") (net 11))
 (segment (start 68.504339 66.354339) (end 68.504339 66.345661) (width 0.2) (layer "B.Cu") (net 11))
 (segment (start 69.05 66.9) (end 68.504339 66.354339) (width 0.5) (layer "B.Cu") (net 11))
 (segment (start 71.75 66.4) (end 71.75 68.565978) (width 0.2) (layer "F.Cu") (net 12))
 (segment (start 70.07952 64.72952) (end 71.75 66.4) (width 0.2) (layer "F.Cu") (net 12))
 (segment (start 70.7205 68.192478) (end 70.7205 68.18479) (width 0.2) (layer "F.Cu") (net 12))
 (segment (start 70.3625 61.4) (end 70.07952 61.68298) (width 0.2) (layer "F.Cu") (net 12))
 (segment (start 69.6375 68.95) (end 69.962978 68.95) (width 0.2) (layer "F.Cu") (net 12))
 (segment (start 69.962978 68.95) (end 70.7205 68.192478) (width 0.2) (layer "F.Cu") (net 12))
 (segment (start 71.2375 61.4) (end 70.3625 61.4) (width 0.2) (layer "F.Cu") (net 12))
 (segment (start 70.07952 61.68298) (end 70.07952 64.72952) (width 0.2) (layer "F.Cu") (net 12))
 (segment (start 71.75 68.565978) (end 72.35 69.165978) (width 0.2) (layer "F.Cu") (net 12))
 (segment (start 72.35 69.165978) (end 72.35 69.5) (width 0.2) (layer "F.Cu") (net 12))
 (via (at 71.7795 68.2) (size 0.6) (drill 0.25) (layers "F.Cu" "B.Cu") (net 12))
 (via (at 70.7205 68.18479) (size 0.6) (drill 0.25) (layers "F.Cu" "B.Cu") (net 12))
 (segment (start 70.7205 68.18479) (end 71.76429 68.18479) (width 0.2) (layer "B.Cu") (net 12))
 (segment (start 71.76429 68.18479) (end 71.7795 68.2) (width 0.2) (layer "B.Cu") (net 12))
 (segment (start 69.75 61.3625) (end 69.75 64.866012) (width 0.2) (layer "F.Cu") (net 13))
 (segment (start 71.25 66.366012) (end 71.25 69.3) (width 0.2) (layer "F.Cu") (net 13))
 (segment (start 69.6375 69.45) (end 71 69.45) (width 0.2) (layer "F.Cu") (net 13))
 (segment (start 71.2375 60.75) (end 70.3625 60.75) (width 0.2) (layer "F.Cu") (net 13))
 (segment (start 71.25 69.3) (end 71.05 69.5) (width 0.2) (layer "F.Cu") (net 13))
 (segment (start 69.75 64.866012) (end 71.25 66.366012) (width 0.2) (layer "F.Cu") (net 13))
 (segment (start 71 69.45) (end 71.05 69.5) (width 0.2) (layer "F.Cu") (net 13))
 (segment (start 70.3625 60.75) (end 69.75 61.3625) (width 0.2) (layer "F.Cu") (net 13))
 (segment (start 68.05 63.83) (end 68.02 63.8) (width 0.2) (layer "F.Cu") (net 5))
 (segment (start 64.2 68.07) (end 64.2 67.75) (width 0.2) (layer "F.Cu") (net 5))
 (via (at 64.2 67.75) (size 0.6) (drill 0.25) (layers "F.Cu" "B.Cu") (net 5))
 (segment (start 69.6375 70.6375) (end 69.75 70.75) (width 0.2) (layer "F.Cu") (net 16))
 (segment (start 69.6375 70.45) (end 69.6375 70.6375) (width 0.2) (layer "F.Cu") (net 16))
 (via (at 69.75 70.75) (size 0.6) (drill 0.25) (layers "F.Cu" "B.Cu") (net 16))
 (segment (start 69.75 70.75) (end 69.45 70.45) (width 0.2) (layer "B.Cu") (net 16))
 (segment (start 62.275 66.975) (end 61.6 66.975) (width 0.2) (layer "B.Cu") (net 16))
 (segment (start 69.45 70.45) (end 65.75 70.45) (width 0.2) (layer "B.Cu") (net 16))
 (segment (start 65.75 70.45) (end 62.275 66.975) (width 0.2) (layer "B.Cu") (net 16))
 (segment (start 64.1 76.97) (end 65.2 78.07) (width 0.2) (layer "F.Cu") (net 15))
 (segment (start 69.8875 68.2) (end 69.6375 67.95) (width 0.2) (layer "F.Cu") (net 15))
 (segment (start 69.6375 68.45) (end 69.6375 67.95) (width 0.4) (layer "F.Cu") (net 15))
 (segment (start 64.1375 74.5) (end 64.1 74.5375) (width 0.2) (layer "F.Cu") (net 15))
 (segment (start 69.85 67.7375) (end 69.6375 67.95) (width 0.2) (layer "F.Cu") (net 15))
 (segment (start 69.679511 67.567011) (end 69.679511 66.369511) (width 0.4) (layer "F.Cu") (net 15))
 (segment (start 69.679511 66.369511) (end 69.06 65.75) (width 0.4) (layer "F.Cu") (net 15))
 (segment (start 69.85 67.7375) (end 69.679511 67.567011) (width 0.4) (layer "F.Cu") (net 15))
 (segment (start 64.6 74.5) (end 64.1375 74.5) (width 0.2) (layer "F.Cu") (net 15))
 (segment (start 64.1 74.5375) (end 64.1 76.97) (width 0.2) (layer "F.Cu") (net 15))
 (segment (start 69.06 65.75) (end 69.06 64.79) (width 0.4) (layer "F.Cu") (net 15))
 (segment (start 69.06 64.79) (end 69.01 64.74) (width 0.4) (layer "F.Cu") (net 15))
 (segment (start 69.9 68.2) (end 69.8875 68.2) (width 0.2) (layer "F.Cu") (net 15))
 (via (at 64.6 74.5) (size 0.6) (drill 0.25) (layers "F.Cu" "B.Cu") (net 15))
 (via (at 69.9 68.2) (size 0.6) (drill 0.25) (layers "F.Cu" "B.Cu") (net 15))
 (segment (start 70.65 71.333988) (end 70.65 68.95) (width 0.2) (layer "B.Cu") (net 15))
 (segment (start 65.9 73.2) (end 68.783988 73.2) (width 0.2) (layer "B.Cu") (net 15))
 (segment (start 70.65 68.95) (end 69.9 68.2) (width 0.2) (layer "B.Cu") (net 15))
 (segment (start 68.783988 73.2) (end 70.65 71.333988) (width 0.2) (layer "B.Cu") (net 15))
 (segment (start 64.6 74.5) (end 65.9 73.2) (width 0.2) (layer "B.Cu") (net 15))
 (segment (start 67.94 67.2525) (end 67.95 67.2625) (width 0.25) (layer "F.Cu") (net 17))
 (segment (start 67.95 65.84) (end 67.95 66.7) (width 0.2) (layer "F.Cu") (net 17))
 (segment (start 67.95 66.36) (end 67.95 66.7) (width 0.2) (layer "F.Cu") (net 17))
 (segment (start 67.95 66.7) (end 67.95 67.2625) (width 0.2) (layer "F.Cu") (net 17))
 (segment (start 68.04 65.75) (end 67.95 65.84) (width 0.2) (layer "F.Cu") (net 17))
 (segment (start 66.95 66.639308) (end 67.069654 66.519654) (width 0.2) (layer "F.Cu") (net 10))
 (segment (start 66.95 67.2625) (end 66.95 66.639308) (width 0.2) (layer "F.Cu") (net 10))
 (via (at 67.069654 66.519654) (size 0.6) (drill 0.25) (layers "F.Cu" "B.Cu") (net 10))
 (segment (start 67.069654 66.519654) (end 67.069654 58.749654) (width 0.2) (layer "B.Cu") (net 10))
 (segment (start 67.069654 58.749654) (end 65.2 56.88) (width 0.2) (layer "B.Cu") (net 10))
 (segment (start 66.95 65.89048) (end 66.95 61.17) (width 0.2) (layer "F.Cu") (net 9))
 (segment (start 66.45 67.2625) (end 66.45 66.39048) (width 0.2) (layer "F.Cu") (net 9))
 (segment (start 66.95 61.17) (end 65.2 59.42) (width 0.2) (layer "F.Cu") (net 9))
 (segment (start 66.45 66.39048) (end 66.95 65.89048) (width 0.2) (layer "F.Cu") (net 9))
 (segment (start 65.7625 66.4875) (end 66.5 65.75) (width 0.2) (layer "F.Cu") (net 8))
 (segment (start 65.7625 67.95) (end 65.7625 66.4875) (width 0.2) (layer "F.Cu") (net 8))
 (segment (start 66.5 63.26) (end 65.2 61.96) (width 0.2) (layer "F.Cu") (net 8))
 (segment (start 66.5 65.75) (end 66.5 63.26) (width 0.2) (layer "F.Cu") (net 8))
 (segment (start 65.1 64.6) (end 65.2 64.5) (width 0.2) (layer "F.Cu") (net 7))
 (segment (start 65.7625 68.45) (end 65.61702 68.59548) (width 0.2) (layer "F.Cu") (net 7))
 (segment (start 65.1 68.146966) (end 65.1 64.6) (width 0.2) (layer "F.Cu") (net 7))
 (segment (start 65.548514 68.59548) (end 65.1 68.146966) (width 0.2) (layer "F.Cu") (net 7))
 (segment (start 65.61702 68.59548) (end 65.548514 68.59548) (width 0.2) (layer "F.Cu") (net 7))
 (segment (start 63.95 61.705) (end 61.6 59.355) (width 0.2) (layer "F.Cu") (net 19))
 (segment (start 63.95 65.85) (end 63.95 61.705) (width 0.2) (layer "F.Cu") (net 19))
 (segment (start 65.7625 68.95) (end 65.437023 68.95) (width 0.2) (layer "F.Cu") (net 19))
 (segment (start 65.437023 68.95) (end 64.77048 68.283457) (width 0.2) (layer "F.Cu") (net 19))
 (segment (start 64.77048 66.67048) (end 63.95 65.85) (width 0.2) (layer "F.Cu") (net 19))
 (segment (start 64.77048 68.283457) (end 64.77048 66.67048) (width 0.2) (layer "F.Cu") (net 19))
 (segment (start 64.62 69.45) (end 65.7625 69.45) (width 0.2) (layer "F.Cu") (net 20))
 (segment (start 64.2 69.03) (end 64.62 69.45) (width 0.2) (layer "F.Cu") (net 20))
 (segment (start 65.7625 69.95) (end 65.7125 70) (width 0.2) (layer "F.Cu") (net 21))
 (segment (start 63.45 63.745) (end 61.6 61.895) (width 0.2) (layer "F.Cu") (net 21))
 (segment (start 63.83742 70) (end 63.45 69.61258) (width 0.2) (layer "F.Cu") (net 21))
 (segment (start 65.7125 70) (end 63.83742 70) (width 0.2) (layer "F.Cu") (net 21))
 (segment (start 63.45 69.61258) (end 63.45 63.745) (width 0.2) (layer "F.Cu") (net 21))
 (segment (start 62.535 70.45) (end 61.6 69.515) (width 0.2) (layer "F.Cu") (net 22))
 (segment (start 65.7625 70.45) (end 62.535 70.45) (width 0.2) (layer "F.Cu") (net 22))
 (segment (start 61.905 71.75) (end 61.6 72.055) (width 0.25) (layer "F.Cu") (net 23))
 (segment (start 66.45 71.1375) (end 66.2125 70.9) (width 0.2) (layer "F.Cu") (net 23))
 (segment (start 66.2125 70.9) (end 62.755 70.9) (width 0.2) (layer "F.Cu") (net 23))
 (segment (start 62.755 70.9) (end 61.6 72.055) (width 0.2) (layer "F.Cu") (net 23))
 (segment (start 67.74 75.1025) (end 67.1375 74.5) (width 0.2) (layer "F.Cu") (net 2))
 (segment (start 67.65 74.45) (end 67.1875 74.45) (width 0.2) (layer "F.Cu") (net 2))
 (segment (start 72.35 72.05) (end 72.35 71.4) (width 0.2) (layer "F.Cu") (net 2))
 (segment (start 67.74 78.07) (end 67.74 75.1025) (width 0.2) (layer "F.Cu") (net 2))
 (segment (start 67.1375 74.5) (end 66.95 74.3125) (width 0.2) (layer "F.Cu") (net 2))
 (segment (start 66.95 74.3125) (end 66.95 71.1375) (width 0.2) (layer "F.Cu") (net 2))
 (segment (start 67.1875 74.45) (end 67.1375 74.5) (width 0.2) (layer "F.Cu") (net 2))
 (via (at 67.65 74.45) (size 0.6) (drill 0.25) (layers "F.Cu" "B.Cu") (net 2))
 (via (at 72.35 72.05) (size 0.6) (drill 0.25) (layers "F.Cu" "B.Cu") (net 2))
 (segment (start 70 74.45) (end 72.35 72.1) (width 0.2) (layer "B.Cu") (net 2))
 (segment (start 67.65 74.45) (end 70 74.45) (width 0.2) (layer "B.Cu") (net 2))
 (segment (start 72.35 72.1) (end 72.35 72.05) (width 0.2) (layer "B.Cu") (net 2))
 (segment (start 67.45 73.1875) (end 68.7625 74.5) (width 0.2) (layer "F.Cu") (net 4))
 (segment (start 70.28 76.0175) (end 70.28 78.07) (width 0.2) (layer "F.Cu") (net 4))
 (segment (start 68.7625 73.6875) (end 71.05 71.4) (width 0.2) (layer "F.Cu") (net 4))
 (segment (start 67.45 71.1375) (end 67.45 73.1875) (width 0.2) (layer "F.Cu") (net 4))
 (segment (start 68.7625 74.5) (end 70.28 76.0175) (width 0.2) (layer "F.Cu") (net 4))
 (segment (start 68.7625 74.5) (end 68.7625 73.6875) (width 0.2) (layer "F.Cu") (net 4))
 (segment (start 67.95 71.1375) (end 67.95 72.130702) (width 0.2) (layer "F.Cu") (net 24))
 (segment (start 67.95 72.130702) (end 67.9795 72.160202) (width 0.2) (layer "F.Cu") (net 24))
 (via (at 67.9795 72.160202) (size 0.6) (drill 0.25) (layers "F.Cu" "B.Cu") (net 24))
 (segment (start 65.039798 72.160202) (end 62.605 74.595) (width 0.2) (layer "B.Cu") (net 24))
 (segment (start 62.605 74.595) (end 61.6 74.595) (width 0.2) (layer "B.Cu") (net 24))
 (segment (start 67.9795 72.160202) (end 65.039798 72.160202) (width 0.2) (layer "B.Cu") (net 24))
 (segment (start 68.45 71.887282) (end 68.708867 72.146149) (width 0.2) (layer "F.Cu") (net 25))
 (segment (start 68.45 71.1375) (end 68.45 71.887282) (width 0.2) (layer "F.Cu") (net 25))
 (via (at 68.708867 72.146149) (size 0.6) (drill 0.25) (layers "F.Cu" "B.Cu") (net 25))
 (segment (start 68.708867 72.179678) (end 68.198832 72.689713) (width 0.2) (layer "B.Cu") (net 25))
 (segment (start 61.6 76.75) (end 61.6 77.135) (width 0.2) (layer "B.Cu") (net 25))
 (segment (start 68.708867 72.146149) (end 68.708867 72.179678) (width 0.2) (layer "B.Cu") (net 25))
 (segment (start 65.660287 72.689713) (end 61.6 76.75) (width 0.2) (layer "B.Cu") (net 25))
 (segment (start 68.198832 72.689713) (end 65.660287 72.689713) (width 0.2) (layer "B.Cu") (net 25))
 (segment (start 62.9 68.348828) (end 62.9 65.735) (width 0.2) (layer "F.Cu") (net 26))
 (segment (start 62.9 65.735) (end 61.6 64.435) (width 0.2) (layer "F.Cu") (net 26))
 (segment (start 68.95 71.1375) (end 68.95 71.15) (width 0.2) (layer "F.Cu") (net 26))
 (segment (start 68.95 71.15) (end 69.25 71.45) (width 0.2) (layer "F.Cu") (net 26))
 (segment (start 62.900586 68.349414) (end 62.9 68.348828) (width 0.2) (layer "F.Cu") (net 26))
 (via (at 69.1 71.5) (size 0.6) (drill 0.25) (layers "F.Cu" "B.Cu") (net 26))
 (via (at 62.900586 68.349414) (size 0.6) (drill 0.25) (layers "F.Cu" "B.Cu") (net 26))
 (segment (start 62.900586 68.349414) (end 62.900586 68.900586) (width 0.2) (layer "B.Cu") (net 26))
 (segment (start 65.35 71.35) (end 69.15 71.35) (width 0.2) (layer "B.Cu") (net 26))
 (segment (start 69.15 71.35) (end 69.25 71.45) (width 0.2) (layer "B.Cu") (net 26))
 (segment (start 62.900586 68.900586) (end 65.35 71.35) (width 0.2) (layer "B.Cu") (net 26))
 (segment (start 65.5625 73.7225) (end 65.35 73.51) (width 0.2) (layer "F.Cu") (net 1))
 (segment (start 65.5625 74.5) (end 65.5625 73.7225) (width 0.2) (layer "F.Cu") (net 1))
 (segment (start 70.3375 74.5) (end 71.48 74.5) (width 0.2) (layer "F.Cu") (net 3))
 (segment (start 63.89 72.1) (end 63.89 72.7525) (width 0.2) (layer "F.Cu") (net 6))
 (segment (start 63.89 72.7525) (end 64.1 72.9625) (width 0.2) (layer "F.Cu") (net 6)))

